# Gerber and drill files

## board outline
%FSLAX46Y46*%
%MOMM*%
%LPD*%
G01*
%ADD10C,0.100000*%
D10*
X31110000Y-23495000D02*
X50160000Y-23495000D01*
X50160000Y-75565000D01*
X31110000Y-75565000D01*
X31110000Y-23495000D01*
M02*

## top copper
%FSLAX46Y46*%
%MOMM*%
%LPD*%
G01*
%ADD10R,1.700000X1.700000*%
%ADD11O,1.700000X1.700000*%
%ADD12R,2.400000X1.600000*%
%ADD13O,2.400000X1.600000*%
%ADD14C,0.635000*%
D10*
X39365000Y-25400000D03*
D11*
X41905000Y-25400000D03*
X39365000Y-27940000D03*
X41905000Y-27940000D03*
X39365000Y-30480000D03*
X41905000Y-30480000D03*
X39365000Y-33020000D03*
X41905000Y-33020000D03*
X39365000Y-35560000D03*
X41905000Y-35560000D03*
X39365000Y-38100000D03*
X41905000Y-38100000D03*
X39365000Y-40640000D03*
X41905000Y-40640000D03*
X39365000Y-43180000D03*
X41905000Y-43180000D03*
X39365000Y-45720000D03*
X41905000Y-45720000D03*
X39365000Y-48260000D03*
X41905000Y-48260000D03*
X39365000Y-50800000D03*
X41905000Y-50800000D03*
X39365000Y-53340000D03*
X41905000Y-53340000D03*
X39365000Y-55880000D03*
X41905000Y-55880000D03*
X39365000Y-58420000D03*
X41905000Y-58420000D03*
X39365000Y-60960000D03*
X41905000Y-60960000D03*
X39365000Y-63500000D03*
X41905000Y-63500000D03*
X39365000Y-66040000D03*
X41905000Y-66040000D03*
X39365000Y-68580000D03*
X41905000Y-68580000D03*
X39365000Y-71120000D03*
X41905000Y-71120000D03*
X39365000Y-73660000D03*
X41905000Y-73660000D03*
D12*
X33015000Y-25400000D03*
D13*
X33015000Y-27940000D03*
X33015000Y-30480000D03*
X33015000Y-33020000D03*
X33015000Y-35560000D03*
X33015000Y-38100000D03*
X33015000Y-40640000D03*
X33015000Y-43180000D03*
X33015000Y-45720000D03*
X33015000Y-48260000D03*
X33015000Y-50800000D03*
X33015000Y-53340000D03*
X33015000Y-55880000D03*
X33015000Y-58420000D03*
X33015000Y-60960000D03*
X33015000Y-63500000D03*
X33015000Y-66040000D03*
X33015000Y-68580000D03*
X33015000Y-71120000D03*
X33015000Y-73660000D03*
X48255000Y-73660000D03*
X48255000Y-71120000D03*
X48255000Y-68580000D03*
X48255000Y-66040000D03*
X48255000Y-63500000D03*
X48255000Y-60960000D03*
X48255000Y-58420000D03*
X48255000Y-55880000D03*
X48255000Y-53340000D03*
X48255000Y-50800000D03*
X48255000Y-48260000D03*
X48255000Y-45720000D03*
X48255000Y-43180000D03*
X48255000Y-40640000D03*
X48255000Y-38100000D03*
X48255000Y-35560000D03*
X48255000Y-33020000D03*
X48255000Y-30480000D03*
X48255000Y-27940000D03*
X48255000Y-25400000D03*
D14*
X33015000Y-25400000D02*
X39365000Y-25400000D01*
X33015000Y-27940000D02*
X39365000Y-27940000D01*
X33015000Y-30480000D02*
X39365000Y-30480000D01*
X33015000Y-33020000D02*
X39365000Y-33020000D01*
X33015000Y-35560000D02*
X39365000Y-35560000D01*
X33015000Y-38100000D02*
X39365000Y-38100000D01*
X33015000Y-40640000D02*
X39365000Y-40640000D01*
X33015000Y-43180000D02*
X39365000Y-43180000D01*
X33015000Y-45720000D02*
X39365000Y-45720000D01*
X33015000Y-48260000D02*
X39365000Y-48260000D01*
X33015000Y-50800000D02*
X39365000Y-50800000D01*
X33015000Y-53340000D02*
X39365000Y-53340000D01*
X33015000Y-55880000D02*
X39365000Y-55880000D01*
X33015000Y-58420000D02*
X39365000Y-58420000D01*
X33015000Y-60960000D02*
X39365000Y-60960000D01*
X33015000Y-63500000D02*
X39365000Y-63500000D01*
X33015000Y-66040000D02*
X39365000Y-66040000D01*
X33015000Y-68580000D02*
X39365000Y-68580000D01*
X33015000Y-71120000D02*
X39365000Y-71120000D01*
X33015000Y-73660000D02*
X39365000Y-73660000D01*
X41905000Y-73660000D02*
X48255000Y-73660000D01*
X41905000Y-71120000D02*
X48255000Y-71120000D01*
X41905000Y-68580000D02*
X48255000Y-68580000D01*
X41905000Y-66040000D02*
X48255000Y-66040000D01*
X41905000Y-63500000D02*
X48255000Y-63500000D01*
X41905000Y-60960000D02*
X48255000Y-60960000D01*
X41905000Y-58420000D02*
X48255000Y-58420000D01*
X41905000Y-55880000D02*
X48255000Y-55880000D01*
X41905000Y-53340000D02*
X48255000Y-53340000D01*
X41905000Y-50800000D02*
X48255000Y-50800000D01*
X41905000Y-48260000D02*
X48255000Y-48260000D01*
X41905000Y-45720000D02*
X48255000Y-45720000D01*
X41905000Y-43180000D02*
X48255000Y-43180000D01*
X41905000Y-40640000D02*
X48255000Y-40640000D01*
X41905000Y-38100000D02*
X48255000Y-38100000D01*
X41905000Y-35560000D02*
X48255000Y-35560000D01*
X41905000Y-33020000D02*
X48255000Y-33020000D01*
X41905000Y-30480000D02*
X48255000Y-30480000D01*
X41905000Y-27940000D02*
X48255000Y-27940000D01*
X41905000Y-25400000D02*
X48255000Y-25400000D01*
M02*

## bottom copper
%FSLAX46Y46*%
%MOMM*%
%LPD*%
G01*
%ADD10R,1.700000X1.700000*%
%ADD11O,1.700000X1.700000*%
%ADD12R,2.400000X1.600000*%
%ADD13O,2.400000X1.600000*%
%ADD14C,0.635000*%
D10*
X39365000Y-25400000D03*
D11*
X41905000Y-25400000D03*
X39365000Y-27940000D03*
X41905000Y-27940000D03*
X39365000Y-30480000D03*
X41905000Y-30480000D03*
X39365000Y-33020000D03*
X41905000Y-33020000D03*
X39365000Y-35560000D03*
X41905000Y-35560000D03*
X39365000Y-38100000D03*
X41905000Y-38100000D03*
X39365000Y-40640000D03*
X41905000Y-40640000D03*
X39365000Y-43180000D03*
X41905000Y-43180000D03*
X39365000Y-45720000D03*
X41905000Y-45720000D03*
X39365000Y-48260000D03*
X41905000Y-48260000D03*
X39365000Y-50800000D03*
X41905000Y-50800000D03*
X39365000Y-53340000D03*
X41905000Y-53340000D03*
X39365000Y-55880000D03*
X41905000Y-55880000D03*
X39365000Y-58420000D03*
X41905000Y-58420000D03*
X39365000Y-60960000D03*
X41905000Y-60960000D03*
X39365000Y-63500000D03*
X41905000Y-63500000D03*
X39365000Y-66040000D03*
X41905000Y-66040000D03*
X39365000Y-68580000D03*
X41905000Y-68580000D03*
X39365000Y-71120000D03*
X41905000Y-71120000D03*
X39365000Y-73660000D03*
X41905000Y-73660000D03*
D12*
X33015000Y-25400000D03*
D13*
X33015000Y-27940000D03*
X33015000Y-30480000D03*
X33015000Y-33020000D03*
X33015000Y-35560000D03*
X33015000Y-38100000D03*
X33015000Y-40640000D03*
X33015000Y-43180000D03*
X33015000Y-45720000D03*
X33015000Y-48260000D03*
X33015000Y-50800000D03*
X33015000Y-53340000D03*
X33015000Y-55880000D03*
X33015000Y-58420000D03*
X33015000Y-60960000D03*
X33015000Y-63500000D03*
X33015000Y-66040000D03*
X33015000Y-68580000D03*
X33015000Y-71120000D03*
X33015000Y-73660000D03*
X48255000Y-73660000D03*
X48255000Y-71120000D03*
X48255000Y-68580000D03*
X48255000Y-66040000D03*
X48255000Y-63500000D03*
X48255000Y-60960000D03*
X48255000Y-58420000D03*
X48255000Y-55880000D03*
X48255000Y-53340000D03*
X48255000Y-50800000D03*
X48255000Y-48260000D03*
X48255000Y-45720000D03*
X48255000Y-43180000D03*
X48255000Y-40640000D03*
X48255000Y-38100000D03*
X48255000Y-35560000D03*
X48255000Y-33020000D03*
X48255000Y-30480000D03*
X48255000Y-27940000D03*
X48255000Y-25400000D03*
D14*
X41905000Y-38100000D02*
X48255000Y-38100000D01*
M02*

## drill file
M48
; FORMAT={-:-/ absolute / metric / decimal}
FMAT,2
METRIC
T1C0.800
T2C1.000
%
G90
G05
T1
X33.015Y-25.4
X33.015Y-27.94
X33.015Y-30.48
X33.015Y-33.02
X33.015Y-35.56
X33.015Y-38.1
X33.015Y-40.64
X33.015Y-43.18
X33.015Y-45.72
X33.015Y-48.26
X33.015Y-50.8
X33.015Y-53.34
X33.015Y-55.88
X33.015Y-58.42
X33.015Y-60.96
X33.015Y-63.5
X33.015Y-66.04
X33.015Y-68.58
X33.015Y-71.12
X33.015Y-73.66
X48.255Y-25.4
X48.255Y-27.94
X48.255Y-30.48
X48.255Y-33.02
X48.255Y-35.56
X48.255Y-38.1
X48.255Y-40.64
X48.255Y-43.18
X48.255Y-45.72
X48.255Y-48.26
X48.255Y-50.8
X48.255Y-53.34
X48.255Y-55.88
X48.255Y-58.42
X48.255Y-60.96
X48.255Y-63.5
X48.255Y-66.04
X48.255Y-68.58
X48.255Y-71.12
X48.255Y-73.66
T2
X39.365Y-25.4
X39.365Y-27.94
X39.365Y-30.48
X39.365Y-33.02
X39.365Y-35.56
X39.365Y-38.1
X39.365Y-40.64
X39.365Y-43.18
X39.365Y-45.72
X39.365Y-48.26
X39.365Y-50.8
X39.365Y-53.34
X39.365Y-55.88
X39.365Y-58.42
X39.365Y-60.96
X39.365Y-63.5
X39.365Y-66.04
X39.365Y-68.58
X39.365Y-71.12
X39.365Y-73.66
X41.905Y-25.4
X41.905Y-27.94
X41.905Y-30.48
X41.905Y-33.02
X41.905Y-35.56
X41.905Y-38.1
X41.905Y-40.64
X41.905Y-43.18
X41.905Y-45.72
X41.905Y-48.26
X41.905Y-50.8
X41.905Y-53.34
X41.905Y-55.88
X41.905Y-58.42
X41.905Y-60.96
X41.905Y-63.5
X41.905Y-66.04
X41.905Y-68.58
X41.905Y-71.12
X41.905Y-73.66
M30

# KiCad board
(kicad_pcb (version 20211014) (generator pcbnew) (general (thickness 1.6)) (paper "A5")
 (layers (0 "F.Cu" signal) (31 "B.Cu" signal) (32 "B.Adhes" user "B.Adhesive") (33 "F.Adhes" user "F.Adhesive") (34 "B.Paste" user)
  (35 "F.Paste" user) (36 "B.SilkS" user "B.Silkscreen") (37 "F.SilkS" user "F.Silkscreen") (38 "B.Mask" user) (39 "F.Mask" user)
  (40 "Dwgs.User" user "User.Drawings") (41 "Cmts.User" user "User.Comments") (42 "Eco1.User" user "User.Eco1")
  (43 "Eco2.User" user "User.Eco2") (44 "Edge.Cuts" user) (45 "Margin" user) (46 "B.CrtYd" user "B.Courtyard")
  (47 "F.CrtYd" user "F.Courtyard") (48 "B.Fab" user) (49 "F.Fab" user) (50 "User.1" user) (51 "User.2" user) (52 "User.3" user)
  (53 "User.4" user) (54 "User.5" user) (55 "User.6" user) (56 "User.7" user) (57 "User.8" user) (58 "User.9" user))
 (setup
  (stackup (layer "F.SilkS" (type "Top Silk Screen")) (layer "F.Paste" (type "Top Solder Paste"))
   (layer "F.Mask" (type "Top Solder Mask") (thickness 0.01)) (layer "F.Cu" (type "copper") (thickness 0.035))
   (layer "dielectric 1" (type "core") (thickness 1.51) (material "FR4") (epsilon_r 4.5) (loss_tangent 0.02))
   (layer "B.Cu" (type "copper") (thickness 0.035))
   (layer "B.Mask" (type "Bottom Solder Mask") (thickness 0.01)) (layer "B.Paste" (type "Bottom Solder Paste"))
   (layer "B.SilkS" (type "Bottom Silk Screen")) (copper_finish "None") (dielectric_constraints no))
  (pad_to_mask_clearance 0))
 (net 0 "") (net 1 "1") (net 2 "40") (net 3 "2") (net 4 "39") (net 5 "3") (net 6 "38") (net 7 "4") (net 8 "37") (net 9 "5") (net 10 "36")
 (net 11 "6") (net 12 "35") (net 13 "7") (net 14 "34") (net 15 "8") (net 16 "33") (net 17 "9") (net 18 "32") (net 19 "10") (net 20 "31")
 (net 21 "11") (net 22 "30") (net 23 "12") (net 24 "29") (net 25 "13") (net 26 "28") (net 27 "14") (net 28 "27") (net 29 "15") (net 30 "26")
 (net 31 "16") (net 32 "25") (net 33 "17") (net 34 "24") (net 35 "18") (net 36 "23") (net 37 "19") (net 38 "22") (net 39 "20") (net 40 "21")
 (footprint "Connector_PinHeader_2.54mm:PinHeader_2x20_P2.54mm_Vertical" (layer "F.Cu") (at 39.365 25.4)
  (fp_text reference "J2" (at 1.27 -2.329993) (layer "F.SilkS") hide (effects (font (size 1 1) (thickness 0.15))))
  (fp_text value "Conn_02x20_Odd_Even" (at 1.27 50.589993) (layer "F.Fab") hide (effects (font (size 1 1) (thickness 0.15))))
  (pad "1" thru_hole rect (at 0 0) (size 1.7 1.7) (drill 1) (layers *.Cu *.Mask) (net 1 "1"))
  (pad "2" thru_hole oval (at 2.54 0) (size 1.7 1.7) (drill 1) (layers *.Cu *.Mask) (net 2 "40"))
  (pad "3" thru_hole oval (at 0 2.54) (size 1.7 1.7) (drill 1) (layers *.Cu *.Mask) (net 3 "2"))
  (pad "4" thru_hole oval (at 2.54 2.54) (size 1.7 1.7) (drill 1) (layers *.Cu *.Mask) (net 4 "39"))
  (pad "5" thru_hole oval (at 0 5.08) (size 1.7 1.7) (drill 1) (layers *.Cu *.Mask) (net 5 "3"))
  (pad "6" thru_hole oval (at 2.54 5.08) (size 1.7 1.7) (drill 1) (layers *.Cu *.Mask) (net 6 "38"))
  (pad "7" thru_hole oval (at 0 7.62) (size 1.7 1.7) (drill 1) (layers *.Cu *.Mask) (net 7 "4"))
  (pad "8" thru_hole oval (at 2.54 7.62) (size 1.7 1.7) (drill 1) (layers *.Cu *.Mask) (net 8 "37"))
  (pad "9" thru_hole oval (at 0 10.16) (size 1.7 1.7) (drill 1) (layers *.Cu *.Mask) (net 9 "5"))
  (pad "10" thru_hole oval (at 2.54 10.16) (size 1.7 1.7) (drill 1) (layers *.Cu *.Mask) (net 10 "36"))
  (pad "11" thru_hole oval (at 0 12.7) (size 1.7 1.7) (drill 1) (layers *.Cu *.Mask) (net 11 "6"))
  (pad "12" thru_hole oval (at 2.54 12.7) (size 1.7 1.7) (drill 1) (layers *.Cu *.Mask) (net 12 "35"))
  (pad "13" thru_hole oval (at 0 15.24) (size 1.7 1.7) (drill 1) (layers *.Cu *.Mask) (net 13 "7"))
  (pad "14" thru_hole oval (at 2.54 15.24) (size 1.7 1.7) (drill 1) (layers *.Cu *.Mask) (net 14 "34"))
  (pad "15" thru_hole oval (at 0 17.78) (size 1.7 1.7) (drill 1) (layers *.Cu *.Mask) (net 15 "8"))
  (pad "16" thru_hole oval (at 2.54 17.78) (size 1.7 1.7) (drill 1) (layers *.Cu *.Mask) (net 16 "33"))
  (pad "17" thru_hole oval (at 0 20.32) (size 1.7 1.7) (drill 1) (layers *.Cu *.Mask) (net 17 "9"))
  (pad "18" thru_hole oval (at 2.54 20.32) (size 1.7 1.7) (drill 1) (layers *.Cu *.Mask) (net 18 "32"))
  (pad "19" thru_hole oval (at 0 22.86) (size 1.7 1.7) (drill 1) (layers *.Cu *.Mask) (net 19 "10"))
  (pad "20" thru_hole oval (at 2.54 22.86) (size 1.7 1.7) (drill 1) (layers *.Cu *.Mask) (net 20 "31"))
  (pad "21" thru_hole oval (at 0 25.4) (size 1.7 1.7) (drill 1) (layers *.Cu *.Mask) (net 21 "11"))
  (pad "22" thru_hole oval (at 2.54 25.4) (size 1.7 1.7) (drill 1) (layers *.Cu *.Mask) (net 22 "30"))
  (pad "23" thru_hole oval (at 0 27.94) (size 1.7 1.7) (drill 1) (layers *.Cu *.Mask) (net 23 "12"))
  (pad "24" thru_hole oval (at 2.54 27.94) (size 1.7 1.7) (drill 1) (layers *.Cu *.Mask) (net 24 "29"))
  (pad "25" thru_hole oval (at 0 30.48) (size 1.7 1.7) (drill 1) (layers *.Cu *.Mask) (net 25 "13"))
  (pad "26" thru_hole oval (at 2.54 30.48) (size 1.7 1.7) (drill 1) (layers *.Cu *.Mask) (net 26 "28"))
  (pad "27" thru_hole oval (at 0 33.02) (size 1.7 1.7) (drill 1) (layers *.Cu *.Mask) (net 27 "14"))
  (pad "28" thru_hole oval (at 2.54 33.02) (size 1.7 1.7) (drill 1) (layers *.Cu *.Mask) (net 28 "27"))
  (pad "29" thru_hole oval (at 0 35.56) (size 1.7 1.7) (drill 1) (layers *.Cu *.Mask) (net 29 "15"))
  (pad "30" thru_hole oval (at 2.54 35.56) (size 1.7 1.7) (drill 1) (layers *.Cu *.Mask) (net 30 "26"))
  (pad "31" thru_hole oval (at 0 38.1) (size 1.7 1.7) (drill 1) (layers *.Cu *.Mask) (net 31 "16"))
  (pad "32" thru_hole oval (at 2.54 38.1) (size 1.7 1.7) (drill 1) (layers *.Cu *.Mask) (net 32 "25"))
  (pad "33" thru_hole oval (at 0 40.64) (size 1.7 1.7) (drill 1) (layers *.Cu *.Mask) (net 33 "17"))
  (pad "34" thru_hole oval (at 2.54 40.64) (size 1.7 1.7) (drill 1) (layers *.Cu *.Mask) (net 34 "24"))
  (pad "35" thru_hole oval (at 0 43.18) (size 1.7 1.7) (drill 1) (layers *.Cu *.Mask) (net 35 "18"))
  (pad "36" thru_hole oval (at 2.54 43.18) (size 1.7 1.7) (drill 1) (layers *.Cu *.Mask) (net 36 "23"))
  (pad "37" thru_hole oval (at 0 45.72) (size 1.7 1.7) (drill 1) (layers *.Cu *.Mask) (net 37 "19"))
  (pad "38" thru_hole oval (at 2.54 45.72) (size 1.7 1.7) (drill 1) (layers *.Cu *.Mask) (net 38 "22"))
  (pad "39" thru_hole oval (at 0 48.26) (size 1.7 1.7) (drill 1) (layers *.Cu *.Mask) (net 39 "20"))
  (pad "40" thru_hole oval (at 2.54 48.26) (size 1.7 1.7) (drill 1) (layers *.Cu *.Mask) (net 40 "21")))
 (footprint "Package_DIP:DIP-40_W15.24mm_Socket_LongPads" (layer "F.Cu") (at 33.015 25.4)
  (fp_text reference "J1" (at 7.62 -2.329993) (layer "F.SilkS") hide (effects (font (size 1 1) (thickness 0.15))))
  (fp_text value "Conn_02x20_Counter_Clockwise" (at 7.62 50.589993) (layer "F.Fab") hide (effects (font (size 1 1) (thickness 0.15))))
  (pad "1" thru_hole rect (at 0 0) (size 2.4 1.6) (drill 0.8) (layers *.Cu *.Mask) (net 1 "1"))
  (pad "2" thru_hole oval (at 0 2.54) (size 2.4 1.6) (drill 0.8) (layers *.Cu *.Mask) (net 3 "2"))
  (pad "3" thru_hole oval (at 0 5.08) (size 2.4 1.6) (drill 0.8) (layers *.Cu *.Mask) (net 5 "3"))
  (pad "4" thru_hole oval (at 0 7.62) (size 2.4 1.6) (drill 0.8) (layers *.Cu *.Mask) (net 7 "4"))
  (pad "5" thru_hole oval (at 0 10.16) (size 2.4 1.6) (drill 0.8) (layers *.Cu *.Mask) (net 9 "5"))
  (pad "6" thru_hole oval (at 0 12.7) (size 2.4 1.6) (drill 0.8) (layers *.Cu *.Mask) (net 11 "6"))
  (pad "7" thru_hole oval (at 0 15.24) (size 2.4 1.6) (drill 0.8) (layers *.Cu *.Mask) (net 13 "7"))
  (pad "8" thru_hole oval (at 0 17.78) (size 2.4 1.6) (drill 0.8) (layers *.Cu *.Mask) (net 15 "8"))
  (pad "9" thru_hole oval (at 0 20.32) (size 2.4 1.6) (drill 0.8) (layers *.Cu *.Mask) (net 17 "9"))
  (pad "10" thru_hole oval (at 0 22.86) (size 2.4 1.6) (drill 0.8) (layers *.Cu *.Mask) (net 19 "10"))
  (pad "11" thru_hole oval (at 0 25.4) (size 2.4 1.6) (drill 0.8) (layers *.Cu *.Mask) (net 21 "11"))
  (pad "12" thru_hole oval (at 0 27.94) (size 2.4 1.6) (drill 0.8) (layers *.Cu *.Mask) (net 23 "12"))
  (pad "13" thru_hole oval (at 0 30.48) (size 2.4 1.6) (drill 0.8) (layers *.Cu *.Mask) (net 25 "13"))
  (pad "14" thru_hole oval (at 0 33.02) (size 2.4 1.6) (drill 0.8) (layers *.Cu *.Mask) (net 27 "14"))
  (pad "15" thru_hole oval (at 0 35.56) (size 2.4 1.6) (drill 0.8) (layers *.Cu *.Mask) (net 29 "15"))
  (pad "16" thru_hole oval (at 0 38.1) (size 2.4 1.6) (drill 0.8) (layers *.Cu *.Mask) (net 31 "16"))
  (pad "17" thru_hole oval (at 0 40.64) (size 2.4 1.6) (drill 0.8) (layers *.Cu *.Mask) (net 33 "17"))
  (pad "18" thru_hole oval (at 0 43.18) (size 2.4 1.6) (drill 0.8) (layers *.Cu *.Mask) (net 35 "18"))
  (pad "19" thru_hole oval (at 0 45.72) (size 2.4 1.6) (drill 0.8) (layers *.Cu *.Mask) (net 37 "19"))
  (pad "20" thru_hole oval (at 0 48.26) (size 2.4 1.6) (drill 0.8) (layers *.Cu *.Mask) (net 39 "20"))
  (pad "21" thru_hole oval (at 15.24 48.26) (size 2.4 1.6) (drill 0.8) (layers *.Cu *.Mask) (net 40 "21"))
  (pad "22" thru_hole oval (at 15.24 45.72) (size 2.4 1.6) (drill 0.8) (layers *.Cu *.Mask) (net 38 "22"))
  (pad "23" thru_hole oval (at 15.24 43.18) (size 2.4 1.6) (drill 0.8) (layers *.Cu *.Mask) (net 36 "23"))
  (pad "24" thru_hole oval (at 15.24 40.64) (size 2.4 1.6) (drill 0.8) (layers *.Cu *.Mask) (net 34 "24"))
  (pad "25" thru_hole oval (at 15.24 38.1) (size 2.4 1.6) (drill 0.8) (layers *.Cu *.Mask) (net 32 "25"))
  (pad "26" thru_hole oval (at 15.24 35.56) (size 2.4 1.6) (drill 0.8) (layers *.Cu *.Mask) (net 30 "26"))
  (pad "27" thru_hole oval (at 15.24 33.02) (size 2.4 1.6) (drill 0.8) (layers *.Cu *.Mask) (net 28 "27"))
  (pad "28" thru_hole oval (at 15.24 30.48) (size 2.4 1.6) (drill 0.8) (layers *.Cu *.Mask) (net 26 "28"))
  (pad "29" thru_hole oval (at 15.24 27.94) (size 2.4 1.6) (drill 0.8) (layers *.Cu *.Mask) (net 24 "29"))
  (pad "30" thru_hole oval (at 15.24 25.4) (size 2.4 1.6) (drill 0.8) (layers *.Cu *.Mask) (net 22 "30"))
  (pad "31" thru_hole oval (at 15.24 22.86) (size 2.4 1.6) (drill 0.8) (layers *.Cu *.Mask) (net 20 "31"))
  (pad "32" thru_hole oval (at 15.24 20.32) (size 2.4 1.6) (drill 0.8) (layers *.Cu *.Mask) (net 18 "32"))
  (pad "33" thru_hole oval (at 15.24 17.78) (size 2.4 1.6) (drill 0.8) (layers *.Cu *.Mask) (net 16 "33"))
  (pad "34" thru_hole oval (at 15.24 15.24) (size 2.4 1.6) (drill 0.8) (layers *.Cu *.Mask) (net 14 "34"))
  (pad "35" thru_hole oval (at 15.24 12.7) (size 2.4 1.6) (drill 0.8) (layers *.Cu *.Mask) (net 12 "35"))
  (pad "36" thru_hole oval (at 15.24 10.16) (size 2.4 1.6) (drill 0.8) (layers *.Cu *.Mask) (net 10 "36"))
  (pad "37" thru_hole oval (at 15.24 7.62) (size 2.4 1.6) (drill 0.8) (layers *.Cu *.Mask) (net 8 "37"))
  (pad "38" thru_hole oval (at 15.24 5.08) (size 2.4 1.6) (drill 0.8) (layers *.Cu *.Mask) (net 6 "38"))
  (pad "39" thru_hole oval (at 15.24 2.54) (size 2.4 1.6) (drill 0.8) (layers *.Cu *.Mask) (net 4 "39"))
  (pad "40" thru_hole oval (at 15.24 0) (size 2.4 1.6) (drill 0.8) (layers *.Cu *.Mask) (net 2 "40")))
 (gr_rect (start 31.11 23.495) (end 50.16 75.565) (layer "Edge.Cuts") (width 0.1) (fill none))
 (segment (start 33.015 25.4) (end 39.365 25.4) (width 0.635) (layer "F.Cu") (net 1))
 (segment (start 33.015 27.94) (end 39.365 27.94) (width 0.635) (layer "F.Cu") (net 3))
 (segment (start 33.015 30.48) (end 39.365 30.48) (width 0.635) (layer "F.Cu") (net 5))
 (segment (start 33.015 33.02) (end 39.365 33.02) (width 0.635) (layer "F.Cu") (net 7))
 (segment (start 33.015 35.56) (end 39.365 35.56) (width 0.635) (layer "F.Cu") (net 9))
 (segment (start 33.015 38.1) (end 39.365 38.1) (width 0.635) (layer "F.Cu") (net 11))
 (segment (start 33.015 40.64) (end 39.365 40.64) (width 0.635) (layer "F.Cu") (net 13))
 (segment (start 33.015 43.18) (end 39.365 43.18) (width 0.635) (layer "F.Cu") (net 15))
 (segment (start 33.015 45.72) (end 39.365 45.72) (width 0.635) (layer "F.Cu") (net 17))
 (segment (start 33.015 48.26) (end 39.365 48.26) (width 0.635) (layer "F.Cu") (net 19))
 (segment (start 33.015 50.8) (end 39.365 50.8) (width 0.635) (layer "F.Cu") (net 21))
 (segment (start 33.015 53.34) (end 39.365 53.34) (width 0.635) (layer "F.Cu") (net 23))
 (segment (start 33.015 55.88) (end 39.365 55.88) (width 0.635) (layer "F.Cu") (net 25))
 (segment (start 33.015 58.42) (end 39.365 58.42) (width 0.635) (layer "F.Cu") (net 27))
 (segment (start 33.015 60.96) (end 39.365 60.96) (width 0.635) (layer "F.Cu") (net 29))
 (segment (start 33.015 63.5) (end 39.365 63.5) (width 0.635) (layer "F.Cu") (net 31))
 (segment (start 33.015 66.04) (end 39.365 66.04) (width 0.635) (layer "F.Cu") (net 33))
 (segment (start 33.015 68.58) (end 39.365 68.58) (width 0.635) (layer "F.Cu") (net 35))
 (segment (start 33.015 71.12) (end 39.365 71.12) (width 0.635) (layer "F.Cu") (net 37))
 (segment (start 33.015 73.66) (end 39.365 73.66) (width 0.635) (layer "F.Cu") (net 39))
 (segment (start 41.905 73.66) (end 48.255 73.66) (width 0.635) (layer "F.Cu") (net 40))
 (segment (start 41.905 71.12) (end 48.255 71.12) (width 0.635) (layer "F.Cu") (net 38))
 (segment (start 41.905 68.58) (end 48.255 68.58) (width 0.635) (layer "F.Cu") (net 36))
 (segment (start 41.905 66.04) (end 48.255 66.04) (width 0.635) (layer "F.Cu") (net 34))
 (segment (start 41.905 63.5) (end 48.255 63.5) (width 0.635) (layer "F.Cu") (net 32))
 (segment (start 41.905 60.96) (end 48.255 60.96) (width 0.635) (layer "F.Cu") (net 30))
 (segment (start 41.905 58.42) (end 48.255 58.42) (width 0.635) (layer "F.Cu") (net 28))
 (segment (start 41.905 55.88) (end 48.255 55.88) (width 0.635) (layer "F.Cu") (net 26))
 (segment (start 41.905 53.34) (end 48.255 53.34) (width 0.635) (layer "F.Cu") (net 24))
 (segment (start 41.905 50.8) (end 48.255 50.8) (width 0.635) (layer "F.Cu") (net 22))
 (segment (start 41.905 48.26) (end 48.255 48.26) (width 0.635) (layer "F.Cu") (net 20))
 (segment (start 41.905 45.72) (end 48.255 45.72) (width 0.635) (layer "F.Cu") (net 18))
 (segment (start 41.905 43.18) (end 48.255 43.18) (width 0.635) (layer "F.Cu") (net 16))
 (segment (start 41.905 40.64) (end 48.255 40.64) (width 0.635) (layer "F.Cu") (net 14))
 (segment (start 41.905 38.1) (end 48.255 38.1) (width 0.635) (layer "F.Cu") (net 12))
 (segment (start 41.905 38.1) (end 48.255 38.1) (width 0.635) (layer "B.Cu") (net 12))
 (segment (start 41.905 35.56) (end 48.255 35.56) (width 0.635) (layer "F.Cu") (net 10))
 (segment (start 41.905 33.02) (end 48.255 33.02) (width 0.635) (layer "F.Cu") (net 8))
 (segment (start 41.905 30.48) (end 48.255 30.48) (width 0.635) (layer "F.Cu") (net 6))
 (segment (start 41.905 27.94) (end 48.255 27.94) (width 0.635) (layer "F.Cu") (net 4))
 (segment (start 41.905 25.4) (end 48.255 25.4) (width 0.635) (layer "F.Cu") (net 2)))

